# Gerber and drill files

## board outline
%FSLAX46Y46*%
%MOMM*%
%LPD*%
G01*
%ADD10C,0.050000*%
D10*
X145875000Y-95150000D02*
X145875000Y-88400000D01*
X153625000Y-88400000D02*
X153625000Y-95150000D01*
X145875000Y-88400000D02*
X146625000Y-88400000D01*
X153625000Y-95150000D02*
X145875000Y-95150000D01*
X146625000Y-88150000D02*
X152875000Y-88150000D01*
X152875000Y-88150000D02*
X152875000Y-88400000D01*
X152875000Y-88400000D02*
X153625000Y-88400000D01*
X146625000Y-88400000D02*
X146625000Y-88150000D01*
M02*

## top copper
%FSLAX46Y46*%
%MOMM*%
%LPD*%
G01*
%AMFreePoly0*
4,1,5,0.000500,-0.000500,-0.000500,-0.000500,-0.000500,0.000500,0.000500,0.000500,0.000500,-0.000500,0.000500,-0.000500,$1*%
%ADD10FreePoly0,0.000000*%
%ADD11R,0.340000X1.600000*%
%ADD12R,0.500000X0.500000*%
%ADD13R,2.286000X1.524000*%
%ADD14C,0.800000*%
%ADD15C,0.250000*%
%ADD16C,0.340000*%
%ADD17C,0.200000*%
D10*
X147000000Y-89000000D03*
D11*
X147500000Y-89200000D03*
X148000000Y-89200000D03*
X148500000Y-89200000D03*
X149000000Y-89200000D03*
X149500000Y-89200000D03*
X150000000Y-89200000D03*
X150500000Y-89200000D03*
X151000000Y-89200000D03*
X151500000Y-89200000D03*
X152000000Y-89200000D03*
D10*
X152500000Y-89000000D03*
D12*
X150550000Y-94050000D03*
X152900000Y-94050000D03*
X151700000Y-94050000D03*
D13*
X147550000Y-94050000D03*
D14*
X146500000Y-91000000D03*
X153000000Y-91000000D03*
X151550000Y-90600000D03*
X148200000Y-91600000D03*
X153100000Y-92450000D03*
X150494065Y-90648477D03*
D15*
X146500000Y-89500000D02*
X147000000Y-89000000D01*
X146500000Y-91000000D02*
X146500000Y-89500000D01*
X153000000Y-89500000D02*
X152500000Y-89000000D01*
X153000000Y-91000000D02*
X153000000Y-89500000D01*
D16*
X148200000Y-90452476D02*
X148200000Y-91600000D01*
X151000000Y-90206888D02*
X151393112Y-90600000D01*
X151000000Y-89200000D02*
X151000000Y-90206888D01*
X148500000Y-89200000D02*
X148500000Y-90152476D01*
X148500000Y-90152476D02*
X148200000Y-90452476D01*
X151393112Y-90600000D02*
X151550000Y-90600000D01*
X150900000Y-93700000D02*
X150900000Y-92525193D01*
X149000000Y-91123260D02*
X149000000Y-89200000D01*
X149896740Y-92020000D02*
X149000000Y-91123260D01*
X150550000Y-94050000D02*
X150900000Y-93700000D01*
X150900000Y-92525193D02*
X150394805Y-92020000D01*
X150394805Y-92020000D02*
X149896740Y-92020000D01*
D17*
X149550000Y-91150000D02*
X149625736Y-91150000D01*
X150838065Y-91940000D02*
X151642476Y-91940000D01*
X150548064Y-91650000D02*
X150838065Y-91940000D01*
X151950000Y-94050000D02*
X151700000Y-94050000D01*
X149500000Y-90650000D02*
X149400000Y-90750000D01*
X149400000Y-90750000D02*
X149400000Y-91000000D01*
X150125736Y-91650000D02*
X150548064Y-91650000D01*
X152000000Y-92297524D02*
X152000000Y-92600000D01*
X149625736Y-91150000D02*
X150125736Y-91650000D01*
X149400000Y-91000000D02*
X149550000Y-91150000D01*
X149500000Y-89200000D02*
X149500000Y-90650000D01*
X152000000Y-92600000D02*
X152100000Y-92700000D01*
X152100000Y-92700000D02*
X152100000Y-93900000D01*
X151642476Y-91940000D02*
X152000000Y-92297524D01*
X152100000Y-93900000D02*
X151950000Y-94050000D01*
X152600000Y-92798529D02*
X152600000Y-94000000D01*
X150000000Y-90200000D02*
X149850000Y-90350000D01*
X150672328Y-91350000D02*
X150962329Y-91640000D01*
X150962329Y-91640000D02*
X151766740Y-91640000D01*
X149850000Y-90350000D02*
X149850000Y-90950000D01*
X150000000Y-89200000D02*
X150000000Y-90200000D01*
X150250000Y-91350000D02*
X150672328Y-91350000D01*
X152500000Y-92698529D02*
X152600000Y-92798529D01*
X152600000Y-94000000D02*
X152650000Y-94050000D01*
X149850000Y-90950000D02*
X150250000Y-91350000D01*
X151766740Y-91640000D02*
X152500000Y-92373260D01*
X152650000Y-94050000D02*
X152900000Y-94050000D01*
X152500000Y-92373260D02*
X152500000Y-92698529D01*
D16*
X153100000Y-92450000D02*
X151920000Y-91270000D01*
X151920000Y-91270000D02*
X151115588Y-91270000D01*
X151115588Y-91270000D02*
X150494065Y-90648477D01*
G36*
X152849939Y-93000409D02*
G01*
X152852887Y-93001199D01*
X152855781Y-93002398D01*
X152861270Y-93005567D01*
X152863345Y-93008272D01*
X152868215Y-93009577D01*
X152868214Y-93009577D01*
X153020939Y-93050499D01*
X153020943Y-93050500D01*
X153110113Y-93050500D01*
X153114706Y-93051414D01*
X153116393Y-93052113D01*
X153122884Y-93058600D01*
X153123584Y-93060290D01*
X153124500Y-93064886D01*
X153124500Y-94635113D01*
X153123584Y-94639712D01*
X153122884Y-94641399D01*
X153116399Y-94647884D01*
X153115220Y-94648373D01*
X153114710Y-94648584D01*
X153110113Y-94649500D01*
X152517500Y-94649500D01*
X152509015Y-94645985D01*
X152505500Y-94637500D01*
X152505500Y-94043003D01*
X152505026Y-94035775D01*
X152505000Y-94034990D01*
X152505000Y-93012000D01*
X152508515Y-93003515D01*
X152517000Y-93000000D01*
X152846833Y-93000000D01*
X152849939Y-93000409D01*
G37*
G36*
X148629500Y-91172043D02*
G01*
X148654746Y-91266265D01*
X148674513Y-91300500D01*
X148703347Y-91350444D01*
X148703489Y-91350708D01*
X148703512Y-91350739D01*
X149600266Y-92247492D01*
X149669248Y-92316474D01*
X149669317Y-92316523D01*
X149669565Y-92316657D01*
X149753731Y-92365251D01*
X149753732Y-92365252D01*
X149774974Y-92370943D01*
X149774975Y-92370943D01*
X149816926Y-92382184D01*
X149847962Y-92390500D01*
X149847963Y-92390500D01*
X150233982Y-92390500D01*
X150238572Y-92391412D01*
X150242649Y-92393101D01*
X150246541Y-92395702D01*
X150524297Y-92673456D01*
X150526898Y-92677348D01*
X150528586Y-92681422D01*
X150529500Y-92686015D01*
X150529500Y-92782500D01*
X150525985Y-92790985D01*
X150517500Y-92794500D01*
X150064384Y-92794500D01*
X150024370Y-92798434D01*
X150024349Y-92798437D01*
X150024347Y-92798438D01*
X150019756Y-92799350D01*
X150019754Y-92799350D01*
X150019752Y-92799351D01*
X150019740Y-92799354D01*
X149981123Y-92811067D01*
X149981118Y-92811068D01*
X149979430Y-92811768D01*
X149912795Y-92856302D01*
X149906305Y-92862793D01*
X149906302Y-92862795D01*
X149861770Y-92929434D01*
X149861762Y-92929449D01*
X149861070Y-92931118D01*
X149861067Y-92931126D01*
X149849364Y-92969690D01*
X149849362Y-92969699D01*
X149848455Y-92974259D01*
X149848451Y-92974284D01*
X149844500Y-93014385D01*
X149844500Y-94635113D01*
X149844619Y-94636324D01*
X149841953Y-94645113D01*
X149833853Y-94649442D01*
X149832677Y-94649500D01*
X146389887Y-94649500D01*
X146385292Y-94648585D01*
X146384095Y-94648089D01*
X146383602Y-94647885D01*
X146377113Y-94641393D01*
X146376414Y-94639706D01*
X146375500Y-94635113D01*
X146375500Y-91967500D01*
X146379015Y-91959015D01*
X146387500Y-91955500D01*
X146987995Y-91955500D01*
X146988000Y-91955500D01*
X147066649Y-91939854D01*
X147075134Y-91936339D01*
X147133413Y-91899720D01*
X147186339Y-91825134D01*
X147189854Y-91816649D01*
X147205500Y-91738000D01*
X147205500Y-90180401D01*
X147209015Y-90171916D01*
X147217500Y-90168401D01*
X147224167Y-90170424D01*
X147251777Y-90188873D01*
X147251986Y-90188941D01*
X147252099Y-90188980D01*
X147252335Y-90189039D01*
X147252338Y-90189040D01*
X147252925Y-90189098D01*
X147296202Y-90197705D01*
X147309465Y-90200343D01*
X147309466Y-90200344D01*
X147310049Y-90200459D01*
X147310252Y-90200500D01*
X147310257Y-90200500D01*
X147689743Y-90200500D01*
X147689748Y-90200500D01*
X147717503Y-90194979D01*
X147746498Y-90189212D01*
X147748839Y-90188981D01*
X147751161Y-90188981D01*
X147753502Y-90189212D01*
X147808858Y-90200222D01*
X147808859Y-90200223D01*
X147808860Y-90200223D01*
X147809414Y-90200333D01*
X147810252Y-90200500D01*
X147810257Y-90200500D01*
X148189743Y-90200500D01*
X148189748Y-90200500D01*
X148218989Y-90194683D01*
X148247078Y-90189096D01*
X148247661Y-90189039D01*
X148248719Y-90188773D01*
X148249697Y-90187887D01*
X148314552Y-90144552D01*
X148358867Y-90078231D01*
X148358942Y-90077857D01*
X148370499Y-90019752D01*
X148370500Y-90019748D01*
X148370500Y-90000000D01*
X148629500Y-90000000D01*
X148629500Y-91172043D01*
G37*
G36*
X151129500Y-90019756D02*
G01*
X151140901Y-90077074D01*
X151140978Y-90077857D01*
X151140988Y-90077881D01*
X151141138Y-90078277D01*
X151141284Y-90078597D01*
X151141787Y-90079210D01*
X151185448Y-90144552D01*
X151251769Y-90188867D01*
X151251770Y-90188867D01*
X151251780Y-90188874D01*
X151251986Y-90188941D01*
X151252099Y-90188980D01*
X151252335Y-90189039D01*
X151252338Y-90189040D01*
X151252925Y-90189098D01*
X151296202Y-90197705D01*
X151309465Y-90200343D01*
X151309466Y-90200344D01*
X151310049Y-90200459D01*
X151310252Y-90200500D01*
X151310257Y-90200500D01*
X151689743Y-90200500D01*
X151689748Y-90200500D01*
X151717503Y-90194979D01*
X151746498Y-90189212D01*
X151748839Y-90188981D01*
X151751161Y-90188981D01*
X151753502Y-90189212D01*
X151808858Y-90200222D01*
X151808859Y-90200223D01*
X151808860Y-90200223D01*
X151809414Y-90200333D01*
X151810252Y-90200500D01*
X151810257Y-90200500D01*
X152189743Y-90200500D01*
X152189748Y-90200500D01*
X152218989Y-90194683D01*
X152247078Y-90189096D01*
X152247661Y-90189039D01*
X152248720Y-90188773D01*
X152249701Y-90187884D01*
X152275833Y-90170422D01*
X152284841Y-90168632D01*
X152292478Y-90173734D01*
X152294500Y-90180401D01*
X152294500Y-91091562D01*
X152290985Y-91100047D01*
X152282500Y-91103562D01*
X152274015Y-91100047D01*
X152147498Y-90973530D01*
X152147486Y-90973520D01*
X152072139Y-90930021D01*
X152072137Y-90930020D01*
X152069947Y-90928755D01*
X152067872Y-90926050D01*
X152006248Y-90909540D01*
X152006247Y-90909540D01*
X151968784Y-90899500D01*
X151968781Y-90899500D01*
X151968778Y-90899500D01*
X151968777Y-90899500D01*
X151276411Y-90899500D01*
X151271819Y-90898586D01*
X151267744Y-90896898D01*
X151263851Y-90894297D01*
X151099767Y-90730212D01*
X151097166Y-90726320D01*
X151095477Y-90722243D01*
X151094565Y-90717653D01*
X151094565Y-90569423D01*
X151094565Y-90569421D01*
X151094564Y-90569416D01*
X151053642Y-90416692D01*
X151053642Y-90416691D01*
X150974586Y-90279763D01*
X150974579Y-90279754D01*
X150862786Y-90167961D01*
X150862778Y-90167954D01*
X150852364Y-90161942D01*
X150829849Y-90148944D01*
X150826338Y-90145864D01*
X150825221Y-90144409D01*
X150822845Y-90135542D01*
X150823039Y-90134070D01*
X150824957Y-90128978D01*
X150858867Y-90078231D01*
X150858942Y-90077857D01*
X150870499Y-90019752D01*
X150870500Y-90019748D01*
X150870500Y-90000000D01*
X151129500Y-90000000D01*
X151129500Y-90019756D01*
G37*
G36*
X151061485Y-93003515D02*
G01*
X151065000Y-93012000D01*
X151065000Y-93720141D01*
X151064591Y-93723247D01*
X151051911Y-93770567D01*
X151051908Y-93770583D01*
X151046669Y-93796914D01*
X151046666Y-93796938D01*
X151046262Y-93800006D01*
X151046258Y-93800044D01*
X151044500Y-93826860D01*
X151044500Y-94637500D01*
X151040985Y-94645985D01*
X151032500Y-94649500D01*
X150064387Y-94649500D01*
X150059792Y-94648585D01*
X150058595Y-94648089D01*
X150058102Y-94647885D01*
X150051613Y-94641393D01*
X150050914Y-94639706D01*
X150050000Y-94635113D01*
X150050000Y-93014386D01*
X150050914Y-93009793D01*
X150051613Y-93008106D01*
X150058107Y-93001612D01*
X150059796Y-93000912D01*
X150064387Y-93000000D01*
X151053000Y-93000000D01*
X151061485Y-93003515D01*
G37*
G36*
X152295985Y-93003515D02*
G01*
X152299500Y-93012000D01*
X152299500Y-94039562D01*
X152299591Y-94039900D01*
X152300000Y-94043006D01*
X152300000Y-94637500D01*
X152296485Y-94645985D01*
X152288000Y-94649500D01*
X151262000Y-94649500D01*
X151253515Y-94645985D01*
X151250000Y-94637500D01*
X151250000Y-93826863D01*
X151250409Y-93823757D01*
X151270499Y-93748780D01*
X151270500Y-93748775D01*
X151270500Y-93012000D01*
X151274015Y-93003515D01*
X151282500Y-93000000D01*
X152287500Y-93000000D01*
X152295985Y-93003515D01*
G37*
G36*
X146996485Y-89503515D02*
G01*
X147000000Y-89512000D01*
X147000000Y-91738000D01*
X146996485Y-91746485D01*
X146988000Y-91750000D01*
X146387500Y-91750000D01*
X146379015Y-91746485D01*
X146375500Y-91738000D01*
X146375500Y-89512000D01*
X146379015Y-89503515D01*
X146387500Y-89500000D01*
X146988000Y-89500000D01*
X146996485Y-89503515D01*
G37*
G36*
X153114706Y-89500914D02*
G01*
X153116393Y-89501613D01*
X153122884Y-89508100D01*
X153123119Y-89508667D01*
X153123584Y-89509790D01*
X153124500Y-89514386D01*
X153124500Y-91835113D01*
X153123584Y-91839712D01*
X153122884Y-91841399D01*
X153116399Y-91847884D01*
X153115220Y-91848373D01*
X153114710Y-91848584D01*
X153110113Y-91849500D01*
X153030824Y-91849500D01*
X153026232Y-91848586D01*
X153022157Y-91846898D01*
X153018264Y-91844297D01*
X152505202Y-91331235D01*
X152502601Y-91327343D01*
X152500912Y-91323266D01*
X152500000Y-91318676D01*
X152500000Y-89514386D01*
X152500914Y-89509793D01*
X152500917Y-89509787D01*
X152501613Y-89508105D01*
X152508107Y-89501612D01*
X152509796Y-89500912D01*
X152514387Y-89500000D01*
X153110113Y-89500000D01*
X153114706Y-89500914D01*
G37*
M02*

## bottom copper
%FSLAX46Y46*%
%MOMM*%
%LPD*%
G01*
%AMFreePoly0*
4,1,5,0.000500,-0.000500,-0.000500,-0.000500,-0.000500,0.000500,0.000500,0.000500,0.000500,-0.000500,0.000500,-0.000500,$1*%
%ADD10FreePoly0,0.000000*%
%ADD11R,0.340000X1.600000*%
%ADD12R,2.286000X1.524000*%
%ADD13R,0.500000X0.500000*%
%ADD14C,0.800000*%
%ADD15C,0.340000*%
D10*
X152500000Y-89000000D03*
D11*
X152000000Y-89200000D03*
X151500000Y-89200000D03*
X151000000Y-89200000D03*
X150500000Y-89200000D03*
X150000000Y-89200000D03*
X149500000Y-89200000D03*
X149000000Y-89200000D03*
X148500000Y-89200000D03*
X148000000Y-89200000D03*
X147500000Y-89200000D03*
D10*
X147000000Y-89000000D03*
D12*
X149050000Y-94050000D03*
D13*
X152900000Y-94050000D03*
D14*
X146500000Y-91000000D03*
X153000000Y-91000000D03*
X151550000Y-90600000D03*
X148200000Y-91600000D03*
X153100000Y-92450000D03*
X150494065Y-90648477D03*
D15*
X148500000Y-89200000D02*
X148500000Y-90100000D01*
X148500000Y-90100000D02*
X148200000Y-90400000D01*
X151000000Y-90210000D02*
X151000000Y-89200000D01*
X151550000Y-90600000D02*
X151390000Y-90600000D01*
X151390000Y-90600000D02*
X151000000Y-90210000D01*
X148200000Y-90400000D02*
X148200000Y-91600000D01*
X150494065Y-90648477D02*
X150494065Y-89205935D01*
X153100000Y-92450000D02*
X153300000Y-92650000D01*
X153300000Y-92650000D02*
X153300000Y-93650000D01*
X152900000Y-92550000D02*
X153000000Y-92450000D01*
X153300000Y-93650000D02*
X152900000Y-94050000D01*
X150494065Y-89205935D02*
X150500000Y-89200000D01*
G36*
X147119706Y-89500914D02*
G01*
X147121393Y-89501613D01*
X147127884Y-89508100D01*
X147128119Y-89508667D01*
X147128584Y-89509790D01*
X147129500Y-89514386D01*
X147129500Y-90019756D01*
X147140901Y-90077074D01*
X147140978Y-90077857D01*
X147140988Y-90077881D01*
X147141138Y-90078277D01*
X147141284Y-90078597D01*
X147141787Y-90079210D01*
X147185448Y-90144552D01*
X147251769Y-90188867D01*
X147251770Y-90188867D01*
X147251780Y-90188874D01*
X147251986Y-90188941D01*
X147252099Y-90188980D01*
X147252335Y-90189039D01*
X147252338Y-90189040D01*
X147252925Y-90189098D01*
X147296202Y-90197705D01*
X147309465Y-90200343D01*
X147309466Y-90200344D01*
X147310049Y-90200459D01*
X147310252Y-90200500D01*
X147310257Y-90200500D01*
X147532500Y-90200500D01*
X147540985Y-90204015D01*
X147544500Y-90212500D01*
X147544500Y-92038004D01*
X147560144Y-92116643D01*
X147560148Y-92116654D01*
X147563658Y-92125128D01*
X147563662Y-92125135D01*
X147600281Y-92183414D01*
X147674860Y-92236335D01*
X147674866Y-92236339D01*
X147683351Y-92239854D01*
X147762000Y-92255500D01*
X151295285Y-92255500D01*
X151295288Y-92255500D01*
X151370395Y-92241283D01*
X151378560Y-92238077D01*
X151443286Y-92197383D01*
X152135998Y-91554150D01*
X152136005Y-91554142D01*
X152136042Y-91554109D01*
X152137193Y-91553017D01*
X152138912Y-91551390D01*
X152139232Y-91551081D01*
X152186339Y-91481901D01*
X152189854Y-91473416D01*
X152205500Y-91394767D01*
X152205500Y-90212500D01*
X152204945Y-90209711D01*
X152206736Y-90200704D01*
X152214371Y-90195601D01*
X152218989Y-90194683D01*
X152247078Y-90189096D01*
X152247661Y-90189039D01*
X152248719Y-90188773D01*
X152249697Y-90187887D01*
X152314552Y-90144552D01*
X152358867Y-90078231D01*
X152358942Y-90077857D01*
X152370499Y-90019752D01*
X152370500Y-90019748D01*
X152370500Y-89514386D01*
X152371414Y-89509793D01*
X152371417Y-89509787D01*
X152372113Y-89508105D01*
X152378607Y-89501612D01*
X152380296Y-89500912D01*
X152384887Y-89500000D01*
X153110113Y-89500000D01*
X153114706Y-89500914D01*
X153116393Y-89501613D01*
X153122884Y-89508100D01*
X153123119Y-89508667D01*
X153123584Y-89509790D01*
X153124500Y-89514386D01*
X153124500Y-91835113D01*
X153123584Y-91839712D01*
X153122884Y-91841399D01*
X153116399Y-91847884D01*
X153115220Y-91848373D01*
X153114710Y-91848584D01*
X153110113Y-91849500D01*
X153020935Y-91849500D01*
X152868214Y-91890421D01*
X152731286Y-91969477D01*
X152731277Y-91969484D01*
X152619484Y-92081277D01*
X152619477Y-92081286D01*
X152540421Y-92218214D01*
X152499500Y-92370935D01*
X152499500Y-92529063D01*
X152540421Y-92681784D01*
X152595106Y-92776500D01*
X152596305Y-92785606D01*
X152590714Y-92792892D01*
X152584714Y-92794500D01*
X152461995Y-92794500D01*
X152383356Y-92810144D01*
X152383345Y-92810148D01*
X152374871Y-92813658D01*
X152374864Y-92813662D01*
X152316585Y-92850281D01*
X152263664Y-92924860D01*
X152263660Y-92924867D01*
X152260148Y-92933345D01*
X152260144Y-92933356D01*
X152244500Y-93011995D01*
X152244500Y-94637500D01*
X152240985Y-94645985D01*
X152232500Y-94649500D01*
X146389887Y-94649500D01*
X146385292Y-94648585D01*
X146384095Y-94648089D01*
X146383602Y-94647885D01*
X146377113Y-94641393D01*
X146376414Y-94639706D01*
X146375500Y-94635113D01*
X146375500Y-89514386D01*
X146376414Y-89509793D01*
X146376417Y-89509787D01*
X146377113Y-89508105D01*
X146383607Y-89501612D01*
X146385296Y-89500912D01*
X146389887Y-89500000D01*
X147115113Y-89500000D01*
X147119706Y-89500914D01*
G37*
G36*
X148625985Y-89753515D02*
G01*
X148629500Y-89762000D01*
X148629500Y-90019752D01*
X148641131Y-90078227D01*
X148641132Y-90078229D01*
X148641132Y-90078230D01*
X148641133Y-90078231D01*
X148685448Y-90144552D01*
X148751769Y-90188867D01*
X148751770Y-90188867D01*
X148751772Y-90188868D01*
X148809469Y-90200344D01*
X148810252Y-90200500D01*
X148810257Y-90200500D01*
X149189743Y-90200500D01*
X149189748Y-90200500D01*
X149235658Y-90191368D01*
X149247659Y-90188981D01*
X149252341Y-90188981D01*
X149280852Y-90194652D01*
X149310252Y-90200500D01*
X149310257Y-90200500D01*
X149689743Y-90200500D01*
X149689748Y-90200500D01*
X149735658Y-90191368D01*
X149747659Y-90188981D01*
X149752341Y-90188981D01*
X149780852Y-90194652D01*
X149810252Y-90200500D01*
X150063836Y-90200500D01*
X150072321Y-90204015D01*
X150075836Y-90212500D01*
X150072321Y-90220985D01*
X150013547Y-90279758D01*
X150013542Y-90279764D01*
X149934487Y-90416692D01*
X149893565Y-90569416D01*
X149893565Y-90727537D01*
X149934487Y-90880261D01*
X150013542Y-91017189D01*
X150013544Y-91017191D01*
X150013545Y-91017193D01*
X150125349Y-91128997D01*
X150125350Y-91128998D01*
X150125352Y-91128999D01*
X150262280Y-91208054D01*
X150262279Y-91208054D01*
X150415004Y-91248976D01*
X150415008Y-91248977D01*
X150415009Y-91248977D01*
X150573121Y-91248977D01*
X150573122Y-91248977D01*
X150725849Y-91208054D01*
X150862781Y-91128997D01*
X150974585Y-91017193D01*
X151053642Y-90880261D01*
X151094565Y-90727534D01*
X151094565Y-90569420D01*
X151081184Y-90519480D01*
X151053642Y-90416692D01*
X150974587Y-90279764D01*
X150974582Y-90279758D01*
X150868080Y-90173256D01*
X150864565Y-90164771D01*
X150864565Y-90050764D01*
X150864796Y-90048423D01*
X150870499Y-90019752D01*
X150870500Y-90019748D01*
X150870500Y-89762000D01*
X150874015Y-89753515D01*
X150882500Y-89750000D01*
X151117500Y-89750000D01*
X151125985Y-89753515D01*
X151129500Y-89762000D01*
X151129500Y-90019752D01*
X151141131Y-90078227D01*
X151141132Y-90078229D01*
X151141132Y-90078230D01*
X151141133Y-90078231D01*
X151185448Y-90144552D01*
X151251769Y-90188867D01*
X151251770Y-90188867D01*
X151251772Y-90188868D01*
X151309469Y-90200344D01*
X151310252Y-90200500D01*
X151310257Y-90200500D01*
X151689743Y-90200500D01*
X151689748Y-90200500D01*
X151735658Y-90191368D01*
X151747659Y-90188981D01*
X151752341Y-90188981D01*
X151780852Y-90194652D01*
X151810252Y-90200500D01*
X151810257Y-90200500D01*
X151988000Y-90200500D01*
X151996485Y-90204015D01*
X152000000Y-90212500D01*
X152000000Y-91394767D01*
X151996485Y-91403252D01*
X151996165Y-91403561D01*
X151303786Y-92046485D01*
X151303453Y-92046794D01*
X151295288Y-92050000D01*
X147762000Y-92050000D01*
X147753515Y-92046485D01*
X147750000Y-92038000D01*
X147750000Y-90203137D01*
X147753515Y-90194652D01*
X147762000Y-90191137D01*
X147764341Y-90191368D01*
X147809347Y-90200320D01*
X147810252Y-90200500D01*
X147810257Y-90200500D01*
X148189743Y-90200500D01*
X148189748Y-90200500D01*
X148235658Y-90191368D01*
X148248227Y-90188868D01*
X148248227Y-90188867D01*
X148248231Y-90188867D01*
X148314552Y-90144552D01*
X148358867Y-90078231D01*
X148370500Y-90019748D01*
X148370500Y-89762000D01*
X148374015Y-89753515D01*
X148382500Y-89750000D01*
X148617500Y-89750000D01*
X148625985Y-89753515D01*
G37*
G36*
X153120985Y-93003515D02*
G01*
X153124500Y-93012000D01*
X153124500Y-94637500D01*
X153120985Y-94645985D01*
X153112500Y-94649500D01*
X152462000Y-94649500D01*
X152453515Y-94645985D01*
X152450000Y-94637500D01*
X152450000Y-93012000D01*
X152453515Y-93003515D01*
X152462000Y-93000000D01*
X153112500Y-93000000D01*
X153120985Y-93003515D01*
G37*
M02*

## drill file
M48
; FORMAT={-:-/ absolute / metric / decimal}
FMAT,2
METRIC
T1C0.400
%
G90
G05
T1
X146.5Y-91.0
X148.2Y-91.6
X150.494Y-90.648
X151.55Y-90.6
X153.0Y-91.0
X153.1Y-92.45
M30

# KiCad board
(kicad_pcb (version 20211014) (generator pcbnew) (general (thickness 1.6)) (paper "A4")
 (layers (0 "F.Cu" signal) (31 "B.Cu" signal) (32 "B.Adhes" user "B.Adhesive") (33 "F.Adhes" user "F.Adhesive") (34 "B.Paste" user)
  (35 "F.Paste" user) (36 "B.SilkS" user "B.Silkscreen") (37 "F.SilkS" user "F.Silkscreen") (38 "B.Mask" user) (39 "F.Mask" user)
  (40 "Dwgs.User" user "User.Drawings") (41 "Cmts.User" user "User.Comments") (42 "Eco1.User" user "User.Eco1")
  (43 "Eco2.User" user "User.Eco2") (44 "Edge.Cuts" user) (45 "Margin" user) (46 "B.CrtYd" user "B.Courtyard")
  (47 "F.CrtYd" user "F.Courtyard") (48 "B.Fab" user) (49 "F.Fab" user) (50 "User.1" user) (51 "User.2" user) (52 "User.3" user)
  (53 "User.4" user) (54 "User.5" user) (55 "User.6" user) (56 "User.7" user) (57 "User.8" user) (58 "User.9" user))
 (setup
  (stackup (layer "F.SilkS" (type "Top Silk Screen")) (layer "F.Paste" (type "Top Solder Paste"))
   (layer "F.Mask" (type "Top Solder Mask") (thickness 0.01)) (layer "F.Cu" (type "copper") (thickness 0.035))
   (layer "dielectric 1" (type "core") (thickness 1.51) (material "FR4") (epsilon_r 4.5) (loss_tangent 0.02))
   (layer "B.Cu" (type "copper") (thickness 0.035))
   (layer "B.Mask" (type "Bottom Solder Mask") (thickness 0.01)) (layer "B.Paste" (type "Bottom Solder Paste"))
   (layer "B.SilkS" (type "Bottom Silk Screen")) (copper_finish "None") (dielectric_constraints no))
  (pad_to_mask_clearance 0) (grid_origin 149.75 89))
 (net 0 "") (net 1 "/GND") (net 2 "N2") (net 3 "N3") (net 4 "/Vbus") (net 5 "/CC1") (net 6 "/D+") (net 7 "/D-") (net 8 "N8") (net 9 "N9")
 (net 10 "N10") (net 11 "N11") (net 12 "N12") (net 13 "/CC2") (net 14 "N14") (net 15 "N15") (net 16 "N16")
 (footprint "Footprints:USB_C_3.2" (layer "F.Cu") (at 149.75 89)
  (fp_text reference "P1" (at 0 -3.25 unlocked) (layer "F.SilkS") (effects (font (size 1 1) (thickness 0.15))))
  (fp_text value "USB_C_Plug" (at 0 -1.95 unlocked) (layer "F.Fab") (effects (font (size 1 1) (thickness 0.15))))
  (pad "A1" smd custom (at -2.75 0) (size 0.001 0.001) (layers "F.Cu" "F.Paste" "F.Mask") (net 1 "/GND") (solder_mask_margin 0.1)
   (zone_connect 2) (options (clearance outline) (anchor rect)) (primitives))
  (pad "A2" smd rect (at -2.25 0.2) (size 0.34 1.6) (layers "F.Cu" "F.Paste" "F.Mask") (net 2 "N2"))
  (pad "A3" smd rect (at -1.75 0.2) (size 0.34 1.6) (layers "F.Cu" "F.Paste" "F.Mask") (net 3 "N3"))
  (pad "A4" smd rect (at -1.25 0.2) (size 0.34 1.6) (layers "F.Cu" "F.Paste" "F.Mask") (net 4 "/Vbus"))
  (pad "A5" smd rect (at -0.75 0.2) (size 0.34 1.6) (layers "F.Cu" "F.Paste" "F.Mask") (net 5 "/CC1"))
  (pad "A6" smd rect (at -0.25 0.2) (size 0.34 1.6) (layers "F.Cu" "F.Paste" "F.Mask") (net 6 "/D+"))
  (pad "A7" smd rect (at 0.25 0.2) (size 0.34 1.6) (layers "F.Cu" "F.Paste" "F.Mask") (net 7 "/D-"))
  (pad "A8" smd rect (at 0.75 0.2) (size 0.34 1.6) (layers "F.Cu" "F.Paste" "F.Mask") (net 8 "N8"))
  (pad "A9" smd rect (at 1.25 0.2) (size 0.34 1.6) (layers "F.Cu" "F.Paste" "F.Mask") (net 4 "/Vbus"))
  (pad "A10" smd rect (at 1.75 0.2) (size 0.34 1.6) (layers "F.Cu" "F.Paste" "F.Mask") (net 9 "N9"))
  (pad "A11" smd rect (at 2.25 0.2) (size 0.34 1.6) (layers "F.Cu" "F.Paste" "F.Mask") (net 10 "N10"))
  (pad "A12" smd custom (at 2.75 0) (size 0.001 0.001) (layers "F.Cu" "F.Paste" "F.Mask") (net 1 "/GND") (solder_mask_margin 0.1)
   (zone_connect 2) (options (clearance outline) (anchor rect)) (primitives))
  (pad "B1" smd custom (at 2.75 0) (size 0.001 0.001) (layers "B.Cu" "B.Paste" "B.Mask") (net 1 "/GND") (solder_mask_margin 0.1)
   (zone_connect 2) (options (clearance outline) (anchor rect)) (primitives))
  (pad "B2" smd rect (at 2.25 0.2) (size 0.34 1.6) (layers "B.Cu" "B.Paste" "B.Mask") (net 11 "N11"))
  (pad "B3" smd rect (at 1.75 0.2) (size 0.34 1.6) (layers "B.Cu" "B.Paste" "B.Mask") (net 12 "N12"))
  (pad "B4" smd rect (at 1.25 0.2) (size 0.34 1.6) (layers "B.Cu" "B.Paste" "B.Mask") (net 4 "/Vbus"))
  (pad "B5" smd rect (at 0.75 0.2) (size 0.34 1.6) (layers "B.Cu" "B.Paste" "B.Mask") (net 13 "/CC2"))
  (pad "B6" smd rect (at 0.25 0.2) (size 0.34 1.6) (layers "B.Cu" "B.Paste" "B.Mask"))
  (pad "B7" smd rect (at -0.25 0.2) (size 0.34 1.6) (layers "B.Cu" "B.Paste" "B.Mask"))
  (pad "B8" smd rect (at -0.75 0.2) (size 0.34 1.6) (layers "B.Cu" "B.Paste" "B.Mask") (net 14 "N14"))
  (pad "B9" smd rect (at -1.25 0.2) (size 0.34 1.6) (layers "B.Cu" "B.Paste" "B.Mask") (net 4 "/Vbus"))
  (pad "B10" smd rect (at -1.75 0.2) (size 0.34 1.6) (layers "B.Cu" "B.Paste" "B.Mask") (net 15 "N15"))
  (pad "B11" smd rect (at -2.25 0.2) (size 0.34 1.6) (layers "B.Cu" "B.Paste" "B.Mask") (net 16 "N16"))
  (pad "B12" smd custom (at -2.75 0) (size 0.001 0.001) (layers "B.Cu" "B.Paste" "B.Mask") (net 1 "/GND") (solder_mask_margin 0.1)
   (zone_connect 2) (options (clearance outline) (anchor rect)) (primitives)))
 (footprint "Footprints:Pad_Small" (layer "F.Cu") (at 150.55 94.05)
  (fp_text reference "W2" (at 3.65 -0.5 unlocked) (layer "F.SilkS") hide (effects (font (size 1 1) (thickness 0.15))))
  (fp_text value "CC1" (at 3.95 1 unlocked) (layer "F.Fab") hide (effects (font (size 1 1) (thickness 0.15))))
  (pad "1" smd rect (at 0 0) (size 0.5 0.5) (layers "F.Cu" "F.Paste" "F.Mask") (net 5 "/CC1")))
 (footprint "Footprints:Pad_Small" (layer "F.Cu") (at 152.9 94.05)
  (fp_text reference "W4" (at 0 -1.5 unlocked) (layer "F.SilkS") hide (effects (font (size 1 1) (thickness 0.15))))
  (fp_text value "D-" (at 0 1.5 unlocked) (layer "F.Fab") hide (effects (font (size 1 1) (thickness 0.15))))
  (pad "1" smd rect (at 0 0) (size 0.5 0.5) (layers "F.Cu" "F.Paste" "F.Mask") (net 7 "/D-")))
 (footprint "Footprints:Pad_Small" (layer "F.Cu") (at 151.7 94.05)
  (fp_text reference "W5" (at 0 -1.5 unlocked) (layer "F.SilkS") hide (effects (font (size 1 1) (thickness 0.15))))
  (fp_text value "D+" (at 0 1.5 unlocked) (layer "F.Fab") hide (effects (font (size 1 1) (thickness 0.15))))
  (pad "1" smd rect (at 0 0) (size 0.5 0.5) (layers "F.Cu" "F.Paste" "F.Mask") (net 6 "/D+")))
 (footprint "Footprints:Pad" (layer "F.Cu") (at 147.55 94.05)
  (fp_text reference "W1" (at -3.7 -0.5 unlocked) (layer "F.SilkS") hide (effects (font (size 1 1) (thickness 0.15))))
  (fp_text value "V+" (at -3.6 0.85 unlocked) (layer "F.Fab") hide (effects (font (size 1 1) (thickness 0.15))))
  (pad "1" smd rect (at 0 0) (size 2.286 1.524) (layers "F.Cu" "F.Paste" "F.Mask") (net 4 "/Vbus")))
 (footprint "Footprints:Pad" (layer "B.Cu") (at 149.05 94.05 180)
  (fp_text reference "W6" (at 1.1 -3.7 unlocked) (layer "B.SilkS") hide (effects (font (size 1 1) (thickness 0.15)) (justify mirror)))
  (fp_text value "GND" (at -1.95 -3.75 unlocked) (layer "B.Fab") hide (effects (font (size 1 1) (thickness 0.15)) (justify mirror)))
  (pad "1" smd rect (at 0 0 180) (size 2.286 1.524) (layers "B.Cu" "B.Paste" "B.Mask") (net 1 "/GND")))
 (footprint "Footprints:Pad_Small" (layer "B.Cu") (at 152.9 94.05 180)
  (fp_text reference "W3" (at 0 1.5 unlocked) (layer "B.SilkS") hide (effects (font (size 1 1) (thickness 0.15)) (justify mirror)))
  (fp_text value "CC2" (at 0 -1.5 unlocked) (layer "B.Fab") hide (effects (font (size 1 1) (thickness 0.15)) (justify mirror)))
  (pad "1" smd rect (at 0 0 180) (size 0.5 0.5) (layers "B.Cu" "B.Paste" "B.Mask") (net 13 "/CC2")))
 (gr_line (start 145.875 95.15) (end 145.875 88.4) (layer "Edge.Cuts") (width 0.05))
 (gr_line (start 153.625 88.4) (end 153.625 95.15) (layer "Edge.Cuts") (width 0.05))
 (gr_line (start 145.875 88.4) (end 146.625 88.4) (layer "Edge.Cuts") (width 0.05))
 (gr_line (start 153.625 95.15) (end 145.875 95.15) (layer "Edge.Cuts") (width 0.05))
 (gr_line (start 146.625 88.15) (end 152.875 88.15) (layer "Edge.Cuts") (width 0.05))
 (gr_line (start 152.875 88.15) (end 152.875 88.4) (layer "Edge.Cuts") (width 0.05))
 (gr_line (start 152.875 88.4) (end 153.625 88.4) (layer "Edge.Cuts") (width 0.05))
 (gr_line (start 146.625 88.4) (end 146.625 88.15) (layer "Edge.Cuts") (width 0.05))
 (segment (start 146.5 89.5) (end 147 89) (width 0.25) (layer "F.Cu") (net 1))
 (segment (start 146.5 91) (end 146.5 89.5) (width 0.25) (layer "F.Cu") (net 1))
 (segment (start 153 89.5) (end 152.5 89) (width 0.25) (layer "F.Cu") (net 1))
 (segment (start 153 91) (end 153 89.5) (width 0.25) (layer "F.Cu") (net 1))
 (via (at 146.5 91) (size 0.8) (drill 0.4) (layers "F.Cu" "B.Cu") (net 1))
 (via (at 153 91) (size 0.8) (drill 0.4) (layers "F.Cu" "B.Cu") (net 1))
 (segment (start 148.2 90.452476) (end 148.2 91.6) (width 0.34) (layer "F.Cu") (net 4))
 (segment (start 151 90.206888) (end 151.393112 90.6) (width 0.34) (layer "F.Cu") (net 4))
 (segment (start 151 89.2) (end 151 90.206888) (width 0.34) (layer "F.Cu") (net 4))
 (segment (start 148.5 89.2) (end 148.5 90.152476) (width 0.34) (layer "F.Cu") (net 4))
 (segment (start 148.5 90.152476) (end 148.2 90.452476) (width 0.34) (layer "F.Cu") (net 4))
 (segment (start 151.393112 90.6) (end 151.55 90.6) (width 0.34) (layer "F.Cu") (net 4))
 (via (at 151.55 90.6) (size 0.8) (drill 0.4) (layers "F.Cu" "B.Cu") (free) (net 4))
 (via (at 148.2 91.6) (size 0.8) (drill 0.4) (layers "F.Cu" "B.Cu") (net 4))
 (segment (start 148.5 89.2) (end 148.5 90.1) (width 0.34) (layer "B.Cu") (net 4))
 (segment (start 148.5 90.1) (end 148.2 90.4) (width 0.34) (layer "B.Cu") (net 4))
 (segment (start 151 90.21) (end 151 89.2) (width 0.34) (layer "B.Cu") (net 4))
 (segment (start 151.55 90.6) (end 151.39 90.6) (width 0.34) (layer "B.Cu") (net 4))
 (segment (start 151.39 90.6) (end 151 90.21) (width 0.34) (layer "B.Cu") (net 4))
 (segment (start 148.2 90.4) (end 148.2 91.6) (width 0.34) (layer "B.Cu") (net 4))
 (segment (start 150.9 93.7) (end 150.9 92.525193) (width 0.34) (layer "F.Cu") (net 5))
 (segment (start 149 91.12326) (end 149 89.2) (width 0.34) (layer "F.Cu") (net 5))
 (segment (start 149.89674 92.02) (end 149 91.12326) (width 0.34) (layer "F.Cu") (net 5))
 (segment (start 150.55 94.05) (end 150.9 93.7) (width 0.34) (layer "F.Cu") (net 5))
 (segment (start 150.9 92.525193) (end 150.394805 92.02) (width 0.34) (layer "F.Cu") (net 5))
 (segment (start 150.394805 92.02) (end 149.89674 92.02) (width 0.34) (layer "F.Cu") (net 5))
 (segment (start 149.55 91.15) (end 149.625736 91.15) (width 0.2) (layer "F.Cu") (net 6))
 (segment (start 150.838065 91.94) (end 151.642476 91.94) (width 0.2) (layer "F.Cu") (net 6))
 (segment (start 150.548064 91.65) (end 150.838065 91.94) (width 0.2) (layer "F.Cu") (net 6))
 (segment (start 151.95 94.05) (end 151.7 94.05) (width 0.2) (layer "F.Cu") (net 6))
 (segment (start 149.5 90.65) (end 149.4 90.75) (width 0.2) (layer "F.Cu") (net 6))
 (segment (start 149.4 90.75) (end 149.4 91) (width 0.2) (layer "F.Cu") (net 6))
 (segment (start 150.125736 91.65) (end 150.548064 91.65) (width 0.2) (layer "F.Cu") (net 6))
 (segment (start 152 92.297524) (end 152 92.6) (width 0.2) (layer "F.Cu") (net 6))
 (segment (start 149.625736 91.15) (end 150.125736 91.65) (width 0.2) (layer "F.Cu") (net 6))
 (segment (start 149.4 91) (end 149.55 91.15) (width 0.2) (layer "F.Cu") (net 6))
 (segment (start 149.5 89.2) (end 149.5 90.65) (width 0.2) (layer "F.Cu") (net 6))
 (segment (start 152 92.6) (end 152.1 92.7) (width 0.2) (layer "F.Cu") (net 6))
 (segment (start 152.1 92.7) (end 152.1 93.9) (width 0.2) (layer "F.Cu") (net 6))
 (segment (start 151.642476 91.94) (end 152 92.297524) (width 0.2) (layer "F.Cu") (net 6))
 (segment (start 152.1 93.9) (end 151.95 94.05) (width 0.2) (layer "F.Cu") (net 6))
 (segment (start 152.6 92.798529) (end 152.6 94) (width 0.2) (layer "F.Cu") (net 7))
 (segment (start 150 90.2) (end 149.85 90.35) (width 0.2) (layer "F.Cu") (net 7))
 (segment (start 150.672328 91.35) (end 150.962329 91.64) (width 0.2) (layer "F.Cu") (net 7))
 (segment (start 150.962329 91.64) (end 151.76674 91.64) (width 0.2) (layer "F.Cu") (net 7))
 (segment (start 149.85 90.35) (end 149.85 90.95) (width 0.2) (layer "F.Cu") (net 7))
 (segment (start 150 89.2) (end 150 90.2) (width 0.2) (layer "F.Cu") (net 7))
 (segment (start 150.25 91.35) (end 150.672328 91.35) (width 0.2) (layer "F.Cu") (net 7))
 (segment (start 152.5 92.698529) (end 152.6 92.798529) (width 0.2) (layer "F.Cu") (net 7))
 (segment (start 152.6 94) (end 152.65 94.05) (width 0.2) (layer "F.Cu") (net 7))
 (segment (start 149.85 90.95) (end 150.25 91.35) (width 0.2) (layer "F.Cu") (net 7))
 (segment (start 151.76674 91.64) (end 152.5 92.37326) (width 0.2) (layer "F.Cu") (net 7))
 (segment (start 152.65 94.05) (end 152.9 94.05) (width 0.2) (layer "F.Cu") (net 7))
 (segment (start 152.5 92.37326) (end 152.5 92.698529) (width 0.2) (layer "F.Cu") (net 7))
 (segment (start 153.1 92.45) (end 151.92 91.27) (width 0.34) (layer "F.Cu") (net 13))
 (segment (start 151.92 91.27) (end 151.115588 91.27) (width 0.34) (layer "F.Cu") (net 13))
 (segment (start 151.115588 91.27) (end 150.494065 90.648477) (width 0.34) (layer "F.Cu") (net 13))
 (via (at 153.1 92.45) (size 0.8) (drill 0.4) (layers "F.Cu" "B.Cu") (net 13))
 (via (at 150.494065 90.648477) (size 0.8) (drill 0.4) (layers "F.Cu" "B.Cu") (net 13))
 (segment (start 150.494065 90.648477) (end 150.494065 89.205935) (width 0.34) (layer "B.Cu") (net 13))
 (segment (start 153.1 92.45) (end 153.3 92.65) (width 0.34) (layer "B.Cu") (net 13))
 (segment (start 153.3 92.65) (end 153.3 93.65) (width 0.34) (layer "B.Cu") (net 13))
 (segment (start 152.9 92.55) (end 153 92.45) (width 0.34) (layer "B.Cu") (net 13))
 (segment (start 153.3 93.65) (end 152.9 94.05) (width 0.34) (layer "B.Cu") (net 13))
 (segment (start 150.494065 89.205935) (end 150.5 89.2) (width 0.34) (layer "B.Cu") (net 13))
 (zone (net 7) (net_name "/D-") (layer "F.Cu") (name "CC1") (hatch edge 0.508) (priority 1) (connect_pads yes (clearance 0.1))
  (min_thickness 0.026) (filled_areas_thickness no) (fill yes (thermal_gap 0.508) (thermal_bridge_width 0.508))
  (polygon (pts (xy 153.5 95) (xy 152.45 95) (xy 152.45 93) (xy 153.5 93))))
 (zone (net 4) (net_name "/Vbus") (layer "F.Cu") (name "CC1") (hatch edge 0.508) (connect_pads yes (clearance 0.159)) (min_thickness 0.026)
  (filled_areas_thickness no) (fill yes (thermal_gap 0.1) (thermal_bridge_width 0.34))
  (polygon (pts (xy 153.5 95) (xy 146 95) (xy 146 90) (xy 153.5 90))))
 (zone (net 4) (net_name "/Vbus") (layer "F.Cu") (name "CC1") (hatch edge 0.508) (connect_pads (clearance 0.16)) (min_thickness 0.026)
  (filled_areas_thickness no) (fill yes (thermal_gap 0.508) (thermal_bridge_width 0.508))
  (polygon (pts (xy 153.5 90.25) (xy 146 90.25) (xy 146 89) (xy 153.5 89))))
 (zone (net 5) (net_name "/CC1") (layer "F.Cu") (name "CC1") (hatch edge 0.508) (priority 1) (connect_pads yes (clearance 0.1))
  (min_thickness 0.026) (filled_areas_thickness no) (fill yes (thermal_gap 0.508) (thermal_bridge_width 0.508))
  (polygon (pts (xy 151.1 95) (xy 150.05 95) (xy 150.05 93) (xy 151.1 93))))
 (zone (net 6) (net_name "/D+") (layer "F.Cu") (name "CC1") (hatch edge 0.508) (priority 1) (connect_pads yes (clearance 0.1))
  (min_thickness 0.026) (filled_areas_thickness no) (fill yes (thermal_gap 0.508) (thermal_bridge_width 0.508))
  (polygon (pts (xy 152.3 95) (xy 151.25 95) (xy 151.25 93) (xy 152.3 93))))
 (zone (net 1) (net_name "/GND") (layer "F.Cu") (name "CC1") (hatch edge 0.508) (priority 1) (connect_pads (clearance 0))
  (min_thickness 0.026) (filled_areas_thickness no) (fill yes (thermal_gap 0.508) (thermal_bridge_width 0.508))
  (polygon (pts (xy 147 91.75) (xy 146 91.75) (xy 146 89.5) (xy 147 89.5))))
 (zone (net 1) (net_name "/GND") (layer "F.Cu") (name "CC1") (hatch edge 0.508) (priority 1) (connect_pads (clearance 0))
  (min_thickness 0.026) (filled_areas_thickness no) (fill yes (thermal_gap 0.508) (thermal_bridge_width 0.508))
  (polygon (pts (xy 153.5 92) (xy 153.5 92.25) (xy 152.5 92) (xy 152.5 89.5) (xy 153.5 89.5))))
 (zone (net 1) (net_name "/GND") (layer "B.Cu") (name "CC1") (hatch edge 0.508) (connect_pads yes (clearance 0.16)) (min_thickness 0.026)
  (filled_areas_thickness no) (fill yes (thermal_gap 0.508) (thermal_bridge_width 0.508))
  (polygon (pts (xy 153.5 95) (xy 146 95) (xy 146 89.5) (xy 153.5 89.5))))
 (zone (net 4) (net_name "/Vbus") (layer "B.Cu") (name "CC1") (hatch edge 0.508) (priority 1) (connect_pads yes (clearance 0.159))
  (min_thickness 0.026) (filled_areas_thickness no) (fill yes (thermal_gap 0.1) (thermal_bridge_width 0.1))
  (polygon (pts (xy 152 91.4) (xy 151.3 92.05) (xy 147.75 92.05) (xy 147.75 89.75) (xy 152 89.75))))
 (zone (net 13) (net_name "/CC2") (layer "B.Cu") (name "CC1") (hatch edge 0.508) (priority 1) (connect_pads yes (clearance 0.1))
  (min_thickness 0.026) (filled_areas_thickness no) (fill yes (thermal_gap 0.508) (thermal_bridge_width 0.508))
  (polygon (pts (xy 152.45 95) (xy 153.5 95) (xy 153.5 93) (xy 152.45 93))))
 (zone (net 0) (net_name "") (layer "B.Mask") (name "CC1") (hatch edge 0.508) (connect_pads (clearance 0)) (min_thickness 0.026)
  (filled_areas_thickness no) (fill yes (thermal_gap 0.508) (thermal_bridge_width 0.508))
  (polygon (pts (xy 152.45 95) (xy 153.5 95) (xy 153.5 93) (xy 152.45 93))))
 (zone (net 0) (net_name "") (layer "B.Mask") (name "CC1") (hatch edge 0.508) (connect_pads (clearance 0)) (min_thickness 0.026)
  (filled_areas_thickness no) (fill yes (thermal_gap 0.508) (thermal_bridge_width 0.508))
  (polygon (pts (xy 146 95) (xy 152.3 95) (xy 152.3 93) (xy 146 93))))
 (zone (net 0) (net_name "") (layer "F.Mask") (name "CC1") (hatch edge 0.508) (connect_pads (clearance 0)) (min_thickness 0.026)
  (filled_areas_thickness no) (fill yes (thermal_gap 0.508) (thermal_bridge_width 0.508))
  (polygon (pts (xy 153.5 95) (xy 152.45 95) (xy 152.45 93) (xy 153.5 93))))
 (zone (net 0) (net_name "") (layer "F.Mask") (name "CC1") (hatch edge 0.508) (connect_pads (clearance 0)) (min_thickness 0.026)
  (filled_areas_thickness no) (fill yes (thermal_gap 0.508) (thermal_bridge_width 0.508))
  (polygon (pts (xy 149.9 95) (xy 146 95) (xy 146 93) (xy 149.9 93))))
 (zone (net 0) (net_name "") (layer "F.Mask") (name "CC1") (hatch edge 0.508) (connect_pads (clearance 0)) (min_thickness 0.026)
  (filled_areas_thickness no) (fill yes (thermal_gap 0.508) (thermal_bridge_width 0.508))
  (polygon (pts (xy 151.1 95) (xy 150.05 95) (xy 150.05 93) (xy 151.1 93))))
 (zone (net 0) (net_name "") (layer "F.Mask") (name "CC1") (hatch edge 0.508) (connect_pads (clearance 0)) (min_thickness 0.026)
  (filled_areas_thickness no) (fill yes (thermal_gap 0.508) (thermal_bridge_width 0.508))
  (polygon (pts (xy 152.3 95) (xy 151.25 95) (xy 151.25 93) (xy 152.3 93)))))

